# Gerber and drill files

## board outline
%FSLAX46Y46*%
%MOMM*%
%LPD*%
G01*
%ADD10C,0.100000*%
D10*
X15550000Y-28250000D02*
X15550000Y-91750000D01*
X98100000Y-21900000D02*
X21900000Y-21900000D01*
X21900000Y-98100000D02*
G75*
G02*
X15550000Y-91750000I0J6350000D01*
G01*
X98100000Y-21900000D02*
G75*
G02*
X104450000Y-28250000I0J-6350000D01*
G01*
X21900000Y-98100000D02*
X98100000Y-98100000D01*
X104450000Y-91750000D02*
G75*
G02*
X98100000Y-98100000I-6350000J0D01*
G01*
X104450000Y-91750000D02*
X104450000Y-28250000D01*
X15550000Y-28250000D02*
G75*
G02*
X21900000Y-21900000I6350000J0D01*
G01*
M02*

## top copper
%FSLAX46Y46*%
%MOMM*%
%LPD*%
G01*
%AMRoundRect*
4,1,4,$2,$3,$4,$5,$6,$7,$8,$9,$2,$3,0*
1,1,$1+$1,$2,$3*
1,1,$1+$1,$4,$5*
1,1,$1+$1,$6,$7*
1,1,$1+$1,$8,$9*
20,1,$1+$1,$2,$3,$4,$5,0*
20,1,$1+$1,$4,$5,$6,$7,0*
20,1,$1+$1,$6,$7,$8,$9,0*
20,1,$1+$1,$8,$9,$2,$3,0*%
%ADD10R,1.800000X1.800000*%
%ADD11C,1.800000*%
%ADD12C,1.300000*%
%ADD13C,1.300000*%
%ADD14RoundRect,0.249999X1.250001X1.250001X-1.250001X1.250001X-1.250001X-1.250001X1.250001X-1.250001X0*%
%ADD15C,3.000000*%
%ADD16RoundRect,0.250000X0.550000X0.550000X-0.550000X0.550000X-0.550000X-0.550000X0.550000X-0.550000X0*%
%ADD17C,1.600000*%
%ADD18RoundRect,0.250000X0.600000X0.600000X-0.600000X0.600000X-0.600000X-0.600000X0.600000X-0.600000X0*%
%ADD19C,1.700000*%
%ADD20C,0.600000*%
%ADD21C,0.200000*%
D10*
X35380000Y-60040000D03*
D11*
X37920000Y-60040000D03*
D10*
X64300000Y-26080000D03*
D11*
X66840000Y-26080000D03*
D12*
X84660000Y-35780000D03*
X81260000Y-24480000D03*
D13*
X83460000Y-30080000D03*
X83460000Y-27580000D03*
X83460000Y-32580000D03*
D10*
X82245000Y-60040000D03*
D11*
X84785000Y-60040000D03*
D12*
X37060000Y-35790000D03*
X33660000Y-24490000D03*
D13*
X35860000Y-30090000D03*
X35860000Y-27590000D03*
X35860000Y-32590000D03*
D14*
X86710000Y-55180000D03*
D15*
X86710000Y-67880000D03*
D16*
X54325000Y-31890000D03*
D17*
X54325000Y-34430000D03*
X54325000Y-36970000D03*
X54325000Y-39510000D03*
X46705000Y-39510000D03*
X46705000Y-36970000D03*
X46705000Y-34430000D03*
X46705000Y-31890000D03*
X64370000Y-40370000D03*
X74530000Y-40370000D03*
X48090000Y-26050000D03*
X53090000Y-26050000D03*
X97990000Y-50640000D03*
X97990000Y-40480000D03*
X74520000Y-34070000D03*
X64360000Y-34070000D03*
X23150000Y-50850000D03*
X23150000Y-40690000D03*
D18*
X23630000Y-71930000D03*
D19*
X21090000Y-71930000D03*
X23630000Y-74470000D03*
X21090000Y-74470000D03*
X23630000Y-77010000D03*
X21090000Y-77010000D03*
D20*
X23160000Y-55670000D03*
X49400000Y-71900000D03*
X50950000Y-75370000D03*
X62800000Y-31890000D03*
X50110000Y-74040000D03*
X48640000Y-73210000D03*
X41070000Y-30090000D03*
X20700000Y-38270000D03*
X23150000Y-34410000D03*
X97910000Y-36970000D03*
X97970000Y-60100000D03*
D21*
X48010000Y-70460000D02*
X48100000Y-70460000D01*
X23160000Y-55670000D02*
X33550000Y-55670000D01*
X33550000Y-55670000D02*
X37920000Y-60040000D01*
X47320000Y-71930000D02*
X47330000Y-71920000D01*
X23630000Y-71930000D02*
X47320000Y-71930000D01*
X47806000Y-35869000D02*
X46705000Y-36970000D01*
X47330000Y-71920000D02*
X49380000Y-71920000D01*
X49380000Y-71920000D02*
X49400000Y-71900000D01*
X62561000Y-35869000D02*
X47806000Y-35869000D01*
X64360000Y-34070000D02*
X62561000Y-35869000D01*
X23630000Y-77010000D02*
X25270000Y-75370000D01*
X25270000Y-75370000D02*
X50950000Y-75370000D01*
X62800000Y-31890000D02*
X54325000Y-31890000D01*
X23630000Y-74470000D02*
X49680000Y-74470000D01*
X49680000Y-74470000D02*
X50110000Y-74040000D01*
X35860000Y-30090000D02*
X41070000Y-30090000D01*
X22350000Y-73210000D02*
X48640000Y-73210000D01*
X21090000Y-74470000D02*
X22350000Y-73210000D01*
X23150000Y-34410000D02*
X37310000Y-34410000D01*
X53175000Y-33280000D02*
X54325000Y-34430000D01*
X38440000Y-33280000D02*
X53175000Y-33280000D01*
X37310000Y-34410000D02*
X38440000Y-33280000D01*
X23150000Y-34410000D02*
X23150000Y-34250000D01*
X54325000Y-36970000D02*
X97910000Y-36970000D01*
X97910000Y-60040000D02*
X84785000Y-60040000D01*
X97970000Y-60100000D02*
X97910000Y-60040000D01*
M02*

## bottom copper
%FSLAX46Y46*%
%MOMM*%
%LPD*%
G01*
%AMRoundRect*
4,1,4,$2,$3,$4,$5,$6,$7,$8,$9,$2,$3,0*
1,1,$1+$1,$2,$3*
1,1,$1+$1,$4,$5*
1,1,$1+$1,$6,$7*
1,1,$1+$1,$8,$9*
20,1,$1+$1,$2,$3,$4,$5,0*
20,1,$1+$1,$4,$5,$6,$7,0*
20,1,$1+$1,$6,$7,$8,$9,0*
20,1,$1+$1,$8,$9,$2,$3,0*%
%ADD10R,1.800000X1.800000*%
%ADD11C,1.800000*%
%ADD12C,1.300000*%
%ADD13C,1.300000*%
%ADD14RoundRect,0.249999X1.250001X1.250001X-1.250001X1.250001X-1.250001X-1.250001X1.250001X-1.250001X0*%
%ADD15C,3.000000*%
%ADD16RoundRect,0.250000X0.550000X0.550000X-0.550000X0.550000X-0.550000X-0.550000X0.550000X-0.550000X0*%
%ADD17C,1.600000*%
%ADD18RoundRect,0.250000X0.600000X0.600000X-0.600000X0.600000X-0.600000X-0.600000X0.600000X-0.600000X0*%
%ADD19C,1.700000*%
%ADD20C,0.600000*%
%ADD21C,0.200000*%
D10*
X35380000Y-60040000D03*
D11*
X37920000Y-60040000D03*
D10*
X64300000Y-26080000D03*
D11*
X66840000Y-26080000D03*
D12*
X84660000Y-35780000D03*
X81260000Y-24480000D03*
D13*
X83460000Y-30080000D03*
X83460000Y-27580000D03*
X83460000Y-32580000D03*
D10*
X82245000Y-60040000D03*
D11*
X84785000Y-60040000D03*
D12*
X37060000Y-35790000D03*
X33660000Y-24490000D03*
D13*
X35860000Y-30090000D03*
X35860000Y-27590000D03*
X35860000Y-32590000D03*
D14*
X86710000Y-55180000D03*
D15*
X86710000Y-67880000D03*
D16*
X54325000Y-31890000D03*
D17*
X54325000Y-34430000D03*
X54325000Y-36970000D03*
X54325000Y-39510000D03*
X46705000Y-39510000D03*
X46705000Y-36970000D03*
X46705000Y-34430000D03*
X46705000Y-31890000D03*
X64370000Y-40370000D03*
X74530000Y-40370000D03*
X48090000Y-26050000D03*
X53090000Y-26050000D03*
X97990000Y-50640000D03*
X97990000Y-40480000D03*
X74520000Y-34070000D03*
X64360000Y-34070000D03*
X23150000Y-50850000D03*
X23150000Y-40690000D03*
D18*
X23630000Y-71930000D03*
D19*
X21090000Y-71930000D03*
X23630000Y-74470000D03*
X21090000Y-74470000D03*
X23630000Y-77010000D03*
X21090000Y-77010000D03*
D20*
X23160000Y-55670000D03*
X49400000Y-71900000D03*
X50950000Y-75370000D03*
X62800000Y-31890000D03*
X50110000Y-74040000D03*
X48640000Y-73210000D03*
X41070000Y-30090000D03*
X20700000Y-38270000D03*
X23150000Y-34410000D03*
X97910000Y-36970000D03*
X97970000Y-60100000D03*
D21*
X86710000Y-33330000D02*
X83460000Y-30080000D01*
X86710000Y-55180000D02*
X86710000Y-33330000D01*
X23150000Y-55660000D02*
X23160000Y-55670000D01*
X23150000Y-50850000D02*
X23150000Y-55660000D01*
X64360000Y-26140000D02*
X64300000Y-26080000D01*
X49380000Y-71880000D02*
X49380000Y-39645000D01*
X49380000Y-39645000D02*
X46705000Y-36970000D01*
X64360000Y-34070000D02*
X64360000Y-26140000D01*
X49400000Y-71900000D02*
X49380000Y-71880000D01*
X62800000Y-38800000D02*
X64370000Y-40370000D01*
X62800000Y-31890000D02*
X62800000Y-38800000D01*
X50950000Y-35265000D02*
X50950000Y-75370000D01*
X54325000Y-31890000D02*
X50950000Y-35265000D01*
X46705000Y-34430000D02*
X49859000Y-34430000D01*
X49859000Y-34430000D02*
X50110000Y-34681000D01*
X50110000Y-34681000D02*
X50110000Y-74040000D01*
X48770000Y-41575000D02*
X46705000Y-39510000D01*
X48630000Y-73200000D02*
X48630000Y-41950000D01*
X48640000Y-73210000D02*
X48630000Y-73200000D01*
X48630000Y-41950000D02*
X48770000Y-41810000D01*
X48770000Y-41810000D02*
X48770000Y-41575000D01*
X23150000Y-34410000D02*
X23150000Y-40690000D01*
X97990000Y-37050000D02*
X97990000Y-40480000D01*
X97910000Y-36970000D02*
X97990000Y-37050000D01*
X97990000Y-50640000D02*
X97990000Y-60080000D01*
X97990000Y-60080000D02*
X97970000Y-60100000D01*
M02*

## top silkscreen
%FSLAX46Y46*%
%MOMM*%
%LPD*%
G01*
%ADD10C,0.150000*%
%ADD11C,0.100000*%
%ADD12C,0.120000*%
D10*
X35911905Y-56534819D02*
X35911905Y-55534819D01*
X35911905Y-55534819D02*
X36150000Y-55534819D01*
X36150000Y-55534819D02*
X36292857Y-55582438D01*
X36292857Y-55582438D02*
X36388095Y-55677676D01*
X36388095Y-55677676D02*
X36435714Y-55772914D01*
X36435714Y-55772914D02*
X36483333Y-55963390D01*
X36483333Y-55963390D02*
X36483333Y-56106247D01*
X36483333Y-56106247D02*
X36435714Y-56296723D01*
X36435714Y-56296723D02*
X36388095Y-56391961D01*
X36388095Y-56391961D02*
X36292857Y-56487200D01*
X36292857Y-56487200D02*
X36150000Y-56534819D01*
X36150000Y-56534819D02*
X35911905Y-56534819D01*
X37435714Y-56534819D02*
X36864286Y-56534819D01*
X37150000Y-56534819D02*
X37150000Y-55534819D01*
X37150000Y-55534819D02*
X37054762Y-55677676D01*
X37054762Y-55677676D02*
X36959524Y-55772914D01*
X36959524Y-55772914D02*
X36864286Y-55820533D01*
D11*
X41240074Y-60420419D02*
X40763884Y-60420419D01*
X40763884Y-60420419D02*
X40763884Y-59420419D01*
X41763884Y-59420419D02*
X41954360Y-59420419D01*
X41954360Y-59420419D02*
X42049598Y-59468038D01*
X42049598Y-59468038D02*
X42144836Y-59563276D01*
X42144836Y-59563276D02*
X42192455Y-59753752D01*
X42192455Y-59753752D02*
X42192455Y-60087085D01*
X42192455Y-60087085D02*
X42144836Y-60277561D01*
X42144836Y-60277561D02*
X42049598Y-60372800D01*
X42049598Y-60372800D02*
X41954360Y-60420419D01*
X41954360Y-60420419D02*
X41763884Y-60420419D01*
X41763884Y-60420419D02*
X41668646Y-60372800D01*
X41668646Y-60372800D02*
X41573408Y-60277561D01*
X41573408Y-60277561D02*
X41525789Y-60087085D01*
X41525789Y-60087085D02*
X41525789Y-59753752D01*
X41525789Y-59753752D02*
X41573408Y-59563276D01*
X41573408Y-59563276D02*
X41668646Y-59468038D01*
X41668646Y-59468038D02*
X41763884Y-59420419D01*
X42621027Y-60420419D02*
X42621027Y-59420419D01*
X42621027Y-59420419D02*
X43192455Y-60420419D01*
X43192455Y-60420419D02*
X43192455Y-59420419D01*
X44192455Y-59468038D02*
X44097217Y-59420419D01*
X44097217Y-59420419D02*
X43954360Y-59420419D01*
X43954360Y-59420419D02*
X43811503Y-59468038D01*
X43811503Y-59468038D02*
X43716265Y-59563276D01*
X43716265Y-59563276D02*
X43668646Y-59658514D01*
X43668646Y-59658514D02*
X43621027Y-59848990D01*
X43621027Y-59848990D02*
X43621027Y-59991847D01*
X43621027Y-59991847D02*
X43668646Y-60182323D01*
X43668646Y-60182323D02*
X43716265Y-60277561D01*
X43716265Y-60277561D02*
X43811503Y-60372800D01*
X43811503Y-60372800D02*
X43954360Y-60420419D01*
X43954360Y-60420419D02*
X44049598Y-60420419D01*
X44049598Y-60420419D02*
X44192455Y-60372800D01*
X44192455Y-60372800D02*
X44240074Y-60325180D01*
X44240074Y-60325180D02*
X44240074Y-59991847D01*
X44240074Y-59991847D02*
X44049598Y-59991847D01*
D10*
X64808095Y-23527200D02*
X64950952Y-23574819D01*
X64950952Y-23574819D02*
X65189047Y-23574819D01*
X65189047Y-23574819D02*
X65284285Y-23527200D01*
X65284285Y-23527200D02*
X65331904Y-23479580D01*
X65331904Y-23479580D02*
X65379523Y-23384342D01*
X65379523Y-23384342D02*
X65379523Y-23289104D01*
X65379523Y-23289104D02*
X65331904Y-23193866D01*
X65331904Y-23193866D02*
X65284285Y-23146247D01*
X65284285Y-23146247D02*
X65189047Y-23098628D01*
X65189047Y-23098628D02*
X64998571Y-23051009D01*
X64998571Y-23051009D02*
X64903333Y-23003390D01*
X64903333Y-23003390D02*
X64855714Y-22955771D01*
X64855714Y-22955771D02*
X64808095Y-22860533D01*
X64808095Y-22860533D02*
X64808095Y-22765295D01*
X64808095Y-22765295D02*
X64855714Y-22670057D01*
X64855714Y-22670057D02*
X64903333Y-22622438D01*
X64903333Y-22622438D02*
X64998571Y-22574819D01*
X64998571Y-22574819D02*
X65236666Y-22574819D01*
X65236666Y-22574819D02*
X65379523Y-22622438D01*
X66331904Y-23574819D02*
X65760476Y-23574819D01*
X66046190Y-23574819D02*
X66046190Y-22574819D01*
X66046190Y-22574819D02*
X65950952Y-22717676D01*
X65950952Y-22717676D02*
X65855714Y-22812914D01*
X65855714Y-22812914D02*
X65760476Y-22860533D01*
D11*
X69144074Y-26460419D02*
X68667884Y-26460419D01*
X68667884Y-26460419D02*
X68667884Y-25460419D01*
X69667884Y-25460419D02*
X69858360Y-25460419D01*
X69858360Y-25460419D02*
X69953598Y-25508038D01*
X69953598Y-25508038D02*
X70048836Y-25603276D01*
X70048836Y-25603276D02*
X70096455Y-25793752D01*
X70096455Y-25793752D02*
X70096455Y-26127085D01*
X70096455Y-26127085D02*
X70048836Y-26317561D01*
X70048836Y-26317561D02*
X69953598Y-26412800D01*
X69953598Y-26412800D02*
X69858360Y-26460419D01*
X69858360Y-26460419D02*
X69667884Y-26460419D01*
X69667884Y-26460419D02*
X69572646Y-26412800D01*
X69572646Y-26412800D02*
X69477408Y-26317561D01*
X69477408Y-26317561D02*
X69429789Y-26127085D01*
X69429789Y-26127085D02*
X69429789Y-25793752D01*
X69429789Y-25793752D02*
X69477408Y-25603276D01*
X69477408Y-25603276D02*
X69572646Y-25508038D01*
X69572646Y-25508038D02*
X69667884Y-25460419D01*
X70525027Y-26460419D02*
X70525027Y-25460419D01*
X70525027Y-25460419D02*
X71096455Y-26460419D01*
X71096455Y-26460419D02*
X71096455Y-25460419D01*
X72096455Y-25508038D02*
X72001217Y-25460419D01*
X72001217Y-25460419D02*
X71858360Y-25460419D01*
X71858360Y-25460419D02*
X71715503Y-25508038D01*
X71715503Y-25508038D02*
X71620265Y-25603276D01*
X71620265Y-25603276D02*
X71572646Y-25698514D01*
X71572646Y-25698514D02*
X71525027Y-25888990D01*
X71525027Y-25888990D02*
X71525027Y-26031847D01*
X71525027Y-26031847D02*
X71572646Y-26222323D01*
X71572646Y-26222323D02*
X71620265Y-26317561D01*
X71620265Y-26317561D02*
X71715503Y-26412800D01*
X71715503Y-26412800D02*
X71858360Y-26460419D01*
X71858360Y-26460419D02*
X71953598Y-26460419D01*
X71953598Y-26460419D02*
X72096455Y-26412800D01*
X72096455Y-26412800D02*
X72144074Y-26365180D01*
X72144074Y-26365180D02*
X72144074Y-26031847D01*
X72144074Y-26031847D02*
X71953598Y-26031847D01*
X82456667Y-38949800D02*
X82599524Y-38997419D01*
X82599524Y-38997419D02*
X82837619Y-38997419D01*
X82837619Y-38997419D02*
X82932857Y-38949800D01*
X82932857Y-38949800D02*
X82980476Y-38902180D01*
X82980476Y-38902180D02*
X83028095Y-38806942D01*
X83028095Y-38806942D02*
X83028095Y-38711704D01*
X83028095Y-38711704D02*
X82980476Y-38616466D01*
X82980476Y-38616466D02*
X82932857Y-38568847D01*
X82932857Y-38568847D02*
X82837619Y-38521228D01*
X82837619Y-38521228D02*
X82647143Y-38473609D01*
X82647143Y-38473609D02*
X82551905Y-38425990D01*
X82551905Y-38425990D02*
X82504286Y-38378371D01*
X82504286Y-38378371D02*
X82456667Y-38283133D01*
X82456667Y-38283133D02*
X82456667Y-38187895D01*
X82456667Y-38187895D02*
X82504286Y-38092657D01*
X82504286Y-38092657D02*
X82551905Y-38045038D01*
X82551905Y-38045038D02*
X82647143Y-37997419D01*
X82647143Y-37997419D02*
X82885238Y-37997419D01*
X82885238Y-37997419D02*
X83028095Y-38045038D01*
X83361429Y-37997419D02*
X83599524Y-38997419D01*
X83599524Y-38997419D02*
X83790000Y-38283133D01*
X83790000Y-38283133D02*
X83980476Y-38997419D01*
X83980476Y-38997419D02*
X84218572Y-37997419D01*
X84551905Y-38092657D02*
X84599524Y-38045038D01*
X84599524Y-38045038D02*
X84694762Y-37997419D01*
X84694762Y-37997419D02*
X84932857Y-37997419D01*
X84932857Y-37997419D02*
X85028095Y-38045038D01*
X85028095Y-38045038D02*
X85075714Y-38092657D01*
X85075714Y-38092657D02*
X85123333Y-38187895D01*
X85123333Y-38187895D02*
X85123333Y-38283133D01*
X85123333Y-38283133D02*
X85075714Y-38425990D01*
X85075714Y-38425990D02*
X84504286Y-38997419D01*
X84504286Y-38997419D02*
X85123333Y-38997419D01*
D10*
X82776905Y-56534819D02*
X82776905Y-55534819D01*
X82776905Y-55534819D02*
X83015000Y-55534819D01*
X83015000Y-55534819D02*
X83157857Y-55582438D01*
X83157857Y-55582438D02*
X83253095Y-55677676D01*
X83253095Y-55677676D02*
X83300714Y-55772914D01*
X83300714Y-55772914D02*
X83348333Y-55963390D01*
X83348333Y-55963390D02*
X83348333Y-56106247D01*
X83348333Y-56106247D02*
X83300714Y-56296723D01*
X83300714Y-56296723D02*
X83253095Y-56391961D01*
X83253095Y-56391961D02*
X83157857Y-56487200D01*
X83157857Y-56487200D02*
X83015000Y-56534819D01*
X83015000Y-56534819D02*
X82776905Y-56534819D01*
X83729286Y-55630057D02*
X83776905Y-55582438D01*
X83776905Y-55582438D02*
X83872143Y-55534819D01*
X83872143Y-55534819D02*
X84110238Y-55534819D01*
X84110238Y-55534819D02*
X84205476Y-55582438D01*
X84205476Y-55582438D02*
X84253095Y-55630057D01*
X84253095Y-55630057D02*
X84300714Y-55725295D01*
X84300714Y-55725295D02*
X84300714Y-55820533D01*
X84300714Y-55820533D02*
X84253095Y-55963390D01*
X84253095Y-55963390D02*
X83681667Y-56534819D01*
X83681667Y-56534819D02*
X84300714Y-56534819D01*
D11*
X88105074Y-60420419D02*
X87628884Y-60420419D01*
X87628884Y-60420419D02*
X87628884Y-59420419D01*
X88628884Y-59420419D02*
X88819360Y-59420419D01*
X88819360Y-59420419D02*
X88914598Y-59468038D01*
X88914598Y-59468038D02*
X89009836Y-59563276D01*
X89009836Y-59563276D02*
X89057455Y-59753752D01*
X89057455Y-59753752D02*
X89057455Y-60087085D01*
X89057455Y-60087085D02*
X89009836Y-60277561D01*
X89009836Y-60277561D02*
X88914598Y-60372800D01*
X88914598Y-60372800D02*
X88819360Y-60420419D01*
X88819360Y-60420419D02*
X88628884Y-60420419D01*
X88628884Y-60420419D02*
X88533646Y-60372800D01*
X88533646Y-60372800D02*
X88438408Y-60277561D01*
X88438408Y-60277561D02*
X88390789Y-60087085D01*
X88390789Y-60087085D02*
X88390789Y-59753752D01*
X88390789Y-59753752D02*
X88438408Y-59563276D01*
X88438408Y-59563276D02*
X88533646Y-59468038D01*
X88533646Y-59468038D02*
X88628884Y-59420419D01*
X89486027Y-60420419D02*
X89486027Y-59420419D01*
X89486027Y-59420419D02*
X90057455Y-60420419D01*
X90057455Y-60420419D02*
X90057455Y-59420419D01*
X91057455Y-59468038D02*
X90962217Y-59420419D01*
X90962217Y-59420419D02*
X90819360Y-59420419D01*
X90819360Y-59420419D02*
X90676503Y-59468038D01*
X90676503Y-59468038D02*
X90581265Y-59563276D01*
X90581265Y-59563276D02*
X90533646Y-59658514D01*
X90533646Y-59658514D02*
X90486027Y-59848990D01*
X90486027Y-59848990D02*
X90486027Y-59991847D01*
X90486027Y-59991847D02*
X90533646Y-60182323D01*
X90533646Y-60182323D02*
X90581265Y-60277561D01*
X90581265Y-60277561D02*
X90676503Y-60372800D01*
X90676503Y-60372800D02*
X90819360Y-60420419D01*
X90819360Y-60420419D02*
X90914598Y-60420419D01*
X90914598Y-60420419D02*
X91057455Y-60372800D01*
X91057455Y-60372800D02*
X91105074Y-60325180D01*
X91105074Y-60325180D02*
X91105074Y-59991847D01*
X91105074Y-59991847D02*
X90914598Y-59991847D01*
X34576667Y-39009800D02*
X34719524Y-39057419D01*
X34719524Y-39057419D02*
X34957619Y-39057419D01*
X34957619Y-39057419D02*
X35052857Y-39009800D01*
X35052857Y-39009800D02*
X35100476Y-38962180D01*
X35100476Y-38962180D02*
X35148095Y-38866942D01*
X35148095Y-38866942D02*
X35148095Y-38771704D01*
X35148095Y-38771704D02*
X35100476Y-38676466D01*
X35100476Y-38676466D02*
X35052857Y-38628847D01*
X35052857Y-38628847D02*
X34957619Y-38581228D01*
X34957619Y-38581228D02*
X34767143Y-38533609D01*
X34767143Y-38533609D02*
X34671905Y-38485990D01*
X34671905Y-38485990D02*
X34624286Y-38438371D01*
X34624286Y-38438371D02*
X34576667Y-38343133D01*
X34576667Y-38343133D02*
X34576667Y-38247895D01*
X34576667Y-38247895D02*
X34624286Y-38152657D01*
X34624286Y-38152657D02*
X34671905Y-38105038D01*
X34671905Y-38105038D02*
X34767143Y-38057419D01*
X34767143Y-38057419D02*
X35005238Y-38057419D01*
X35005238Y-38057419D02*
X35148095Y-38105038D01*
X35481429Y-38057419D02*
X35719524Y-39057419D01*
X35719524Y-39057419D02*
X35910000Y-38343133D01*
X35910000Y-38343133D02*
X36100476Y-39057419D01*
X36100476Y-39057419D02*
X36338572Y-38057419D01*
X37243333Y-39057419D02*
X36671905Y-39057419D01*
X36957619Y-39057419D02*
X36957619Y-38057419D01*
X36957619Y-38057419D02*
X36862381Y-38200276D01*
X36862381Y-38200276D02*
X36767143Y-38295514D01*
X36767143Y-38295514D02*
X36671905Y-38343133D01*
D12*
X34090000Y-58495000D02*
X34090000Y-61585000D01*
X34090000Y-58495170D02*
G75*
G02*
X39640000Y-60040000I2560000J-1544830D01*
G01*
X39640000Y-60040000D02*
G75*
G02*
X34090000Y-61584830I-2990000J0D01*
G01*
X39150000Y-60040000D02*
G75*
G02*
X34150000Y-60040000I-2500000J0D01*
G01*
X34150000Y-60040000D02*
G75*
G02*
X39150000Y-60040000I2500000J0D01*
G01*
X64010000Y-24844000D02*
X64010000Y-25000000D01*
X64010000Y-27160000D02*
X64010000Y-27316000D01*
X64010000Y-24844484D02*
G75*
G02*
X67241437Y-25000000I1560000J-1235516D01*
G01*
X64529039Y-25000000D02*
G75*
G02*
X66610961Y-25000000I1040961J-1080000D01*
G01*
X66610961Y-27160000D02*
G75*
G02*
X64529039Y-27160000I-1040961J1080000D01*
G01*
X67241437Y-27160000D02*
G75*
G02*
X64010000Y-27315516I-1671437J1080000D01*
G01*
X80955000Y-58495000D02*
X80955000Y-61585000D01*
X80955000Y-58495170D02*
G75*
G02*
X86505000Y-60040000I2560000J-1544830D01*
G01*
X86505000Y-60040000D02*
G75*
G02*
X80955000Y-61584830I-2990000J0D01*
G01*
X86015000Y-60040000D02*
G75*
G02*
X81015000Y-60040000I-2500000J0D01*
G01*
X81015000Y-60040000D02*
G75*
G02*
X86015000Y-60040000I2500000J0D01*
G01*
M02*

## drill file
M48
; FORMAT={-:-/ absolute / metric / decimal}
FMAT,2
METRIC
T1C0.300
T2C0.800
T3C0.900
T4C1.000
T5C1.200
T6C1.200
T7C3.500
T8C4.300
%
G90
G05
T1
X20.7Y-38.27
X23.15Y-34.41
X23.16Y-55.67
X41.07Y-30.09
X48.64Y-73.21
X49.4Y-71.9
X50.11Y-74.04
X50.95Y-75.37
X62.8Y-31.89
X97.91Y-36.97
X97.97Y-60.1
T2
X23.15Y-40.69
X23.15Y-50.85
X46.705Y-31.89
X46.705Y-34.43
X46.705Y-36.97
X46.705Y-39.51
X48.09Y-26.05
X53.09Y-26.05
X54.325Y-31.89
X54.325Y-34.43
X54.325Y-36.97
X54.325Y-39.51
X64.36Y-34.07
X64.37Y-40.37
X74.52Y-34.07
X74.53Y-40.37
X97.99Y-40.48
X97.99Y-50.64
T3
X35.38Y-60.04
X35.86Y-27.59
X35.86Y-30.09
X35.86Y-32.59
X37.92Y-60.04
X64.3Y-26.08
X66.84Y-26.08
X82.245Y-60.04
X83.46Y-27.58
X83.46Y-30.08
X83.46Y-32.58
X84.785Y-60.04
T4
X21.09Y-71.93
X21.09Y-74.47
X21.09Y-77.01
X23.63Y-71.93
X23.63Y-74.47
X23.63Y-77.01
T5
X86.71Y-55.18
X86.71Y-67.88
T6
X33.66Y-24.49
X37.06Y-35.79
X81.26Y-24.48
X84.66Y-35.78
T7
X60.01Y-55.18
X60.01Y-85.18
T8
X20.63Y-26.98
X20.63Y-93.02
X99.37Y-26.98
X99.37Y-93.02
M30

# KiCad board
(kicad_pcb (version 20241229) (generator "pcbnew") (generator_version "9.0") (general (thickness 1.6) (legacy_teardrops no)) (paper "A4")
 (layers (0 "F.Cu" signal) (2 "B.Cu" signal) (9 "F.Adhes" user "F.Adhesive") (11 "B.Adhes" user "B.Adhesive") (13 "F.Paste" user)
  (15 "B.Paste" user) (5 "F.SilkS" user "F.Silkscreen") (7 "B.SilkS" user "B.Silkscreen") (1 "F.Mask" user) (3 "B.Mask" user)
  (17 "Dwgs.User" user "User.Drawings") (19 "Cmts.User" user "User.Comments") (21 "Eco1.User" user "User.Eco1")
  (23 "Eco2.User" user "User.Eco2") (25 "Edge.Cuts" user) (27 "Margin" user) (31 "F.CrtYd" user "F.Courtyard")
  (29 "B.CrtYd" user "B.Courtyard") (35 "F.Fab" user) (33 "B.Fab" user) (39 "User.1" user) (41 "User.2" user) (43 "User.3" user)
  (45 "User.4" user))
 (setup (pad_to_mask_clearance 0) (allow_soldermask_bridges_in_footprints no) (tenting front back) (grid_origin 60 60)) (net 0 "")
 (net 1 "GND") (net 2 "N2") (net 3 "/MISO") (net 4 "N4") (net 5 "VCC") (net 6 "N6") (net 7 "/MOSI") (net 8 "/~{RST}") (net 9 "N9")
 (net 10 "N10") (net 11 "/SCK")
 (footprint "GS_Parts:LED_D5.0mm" (layer "F.Cu") (at 35.38 60.04)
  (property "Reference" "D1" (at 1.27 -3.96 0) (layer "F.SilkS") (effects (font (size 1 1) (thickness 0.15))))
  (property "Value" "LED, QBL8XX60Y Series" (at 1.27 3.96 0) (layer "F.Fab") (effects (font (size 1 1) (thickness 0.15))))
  (fp_line (start -1.29 -1.545) (end -1.29 1.545) (stroke (width 0.12) (type solid)) (layer "F.SilkS"))
  (fp_arc (start -1.29 -1.54483) (mid 2.071779 -2.880495) (end 4.26 0) (stroke (width 0.12) (type solid)) (layer "F.SilkS"))
  (fp_arc (start 4.26 0) (mid 2.071779 2.880495) (end -1.29 1.54483) (stroke (width 0.12) (type solid)) (layer "F.SilkS"))
  (fp_circle (center 1.27 0) (end 3.77 0) (stroke (width 0.12) (type solid)) (fill no) (layer "F.SilkS"))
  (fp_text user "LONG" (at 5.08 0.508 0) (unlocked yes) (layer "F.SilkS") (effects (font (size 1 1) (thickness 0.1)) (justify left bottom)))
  (pad "1" thru_hole rect (at 0 0) (size 1.8 1.8) (drill 0.9) (layers "*.Cu" "*.Mask") (remove_unused_layers no) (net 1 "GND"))
  (pad "2" thru_hole circle (at 2.54 0) (size 1.8 1.8) (drill 0.9) (layers "*.Cu" "*.Mask") (remove_unused_layers no) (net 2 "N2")))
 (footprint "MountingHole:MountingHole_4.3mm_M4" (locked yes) (layer "F.Cu") (at 20.63 26.98 90)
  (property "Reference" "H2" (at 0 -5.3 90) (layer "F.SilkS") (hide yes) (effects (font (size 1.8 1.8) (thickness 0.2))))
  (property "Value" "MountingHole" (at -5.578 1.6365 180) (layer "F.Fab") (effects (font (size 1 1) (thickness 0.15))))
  (pad "" np_thru_hole circle (at 0 0 90) (size 4.3 4.3) (drill 4.3) (layers "*.Cu" "*.Mask")))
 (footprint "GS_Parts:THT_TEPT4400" (layer "F.Cu") (at 64.3 26.08)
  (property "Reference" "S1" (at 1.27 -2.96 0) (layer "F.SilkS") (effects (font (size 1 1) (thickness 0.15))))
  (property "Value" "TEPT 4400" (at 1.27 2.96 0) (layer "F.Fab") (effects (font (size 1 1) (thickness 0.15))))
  (fp_line (start -0.29 -1.236) (end -0.29 -1.08) (stroke (width 0.12) (type solid)) (layer "F.SilkS"))
  (fp_line (start -0.29 1.08) (end -0.29 1.236) (stroke (width 0.12) (type solid)) (layer "F.SilkS"))
  (fp_arc (start -0.29 -1.235516) (mid 1.36566 -1.987699) (end 2.941437 -1.08) (stroke (width 0.12) (type solid)) (layer "F.SilkS"))
  (fp_arc (start 0.229039 -1.08) (mid 1.27 -1.5) (end 2.310961 -1.08) (stroke (width 0.12) (type solid)) (layer "F.SilkS"))
  (fp_arc (start 2.310961 1.08) (mid 1.27 1.5) (end 0.229039 1.08) (stroke (width 0.12) (type solid)) (layer "F.SilkS"))
  (fp_arc (start 2.941437 1.08) (mid 1.36566 1.987699) (end -0.29 1.235516) (stroke (width 0.12) (type solid)) (layer "F.SilkS"))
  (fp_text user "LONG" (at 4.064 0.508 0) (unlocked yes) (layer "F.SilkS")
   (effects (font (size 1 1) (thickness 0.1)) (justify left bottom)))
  (pad "1" thru_hole rect (at 0 0) (size 1.8 1.8) (drill 0.9) (layers "*.Cu" "*.Mask") (remove_unused_layers no) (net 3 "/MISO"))
  (pad "2" thru_hole circle (at 2.54 0) (size 1.8 1.8) (drill 0.9) (layers "*.Cu" "*.Mask") (remove_unused_layers no) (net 1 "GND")))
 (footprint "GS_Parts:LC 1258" (layer "F.Cu") (at 83.46 30.08 90)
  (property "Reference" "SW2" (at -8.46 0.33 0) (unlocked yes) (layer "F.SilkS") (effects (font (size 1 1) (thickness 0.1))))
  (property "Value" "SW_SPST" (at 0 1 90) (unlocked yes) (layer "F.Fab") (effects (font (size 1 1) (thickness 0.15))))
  (pad "" np_thru_hole circle (at -5.7 1.2 90) (size 1.3 1.3) (drill 1.2) (layers "*.Cu" "*.Mask"))
  (pad "" np_thru_hole circle (at 5.6 -2.2 90) (size 1.3 1.3) (drill 1.2) (layers "*.Cu" "*.Mask"))
  (pad "1" thru_hole circle (at 0 0 90) (size 1.3 1.3) (drill 0.9) (layers "*.Cu" "*.Mask") (remove_unused_layers no) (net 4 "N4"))
  (pad "2" thru_hole circle (at 2.5 0 90) (size 1.3 1.3) (drill 0.9) (layers "*.Cu" "*.Mask") (remove_unused_layers no) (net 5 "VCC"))
  (pad "3" thru_hole circle (at -2.5 0 90) (size 1.3 1.3) (drill 0.9) (layers "*.Cu" "*.Mask") (remove_unused_layers no)))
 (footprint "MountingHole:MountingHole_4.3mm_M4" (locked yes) (layer "F.Cu") (at 99.37 93.02 90)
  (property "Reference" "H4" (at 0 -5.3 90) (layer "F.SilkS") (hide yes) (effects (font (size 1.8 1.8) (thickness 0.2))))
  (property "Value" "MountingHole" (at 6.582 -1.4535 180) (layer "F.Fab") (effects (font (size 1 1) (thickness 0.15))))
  (pad "" np_thru_hole circle (at 0 0 90) (size 4.3 4.3) (drill 4.3) (layers "*.Cu" "*.Mask")))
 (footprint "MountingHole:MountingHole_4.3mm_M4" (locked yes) (layer "F.Cu") (at 99.37 26.98 90)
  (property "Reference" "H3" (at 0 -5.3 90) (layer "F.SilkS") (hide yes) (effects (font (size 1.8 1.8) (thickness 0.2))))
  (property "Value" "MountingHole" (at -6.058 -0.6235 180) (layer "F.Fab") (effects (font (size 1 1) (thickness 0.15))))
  (pad "" np_thru_hole circle (at 0 0 90) (size 4.3 4.3) (drill 4.3) (layers "*.Cu" "*.Mask")))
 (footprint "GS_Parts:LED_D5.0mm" (layer "F.Cu") (at 82.245 60.04)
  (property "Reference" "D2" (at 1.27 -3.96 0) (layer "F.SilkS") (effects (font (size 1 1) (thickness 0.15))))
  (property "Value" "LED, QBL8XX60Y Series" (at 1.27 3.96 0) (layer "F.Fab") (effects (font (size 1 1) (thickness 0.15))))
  (fp_line (start -1.29 -1.545) (end -1.29 1.545) (stroke (width 0.12) (type solid)) (layer "F.SilkS"))
  (fp_arc (start -1.29 -1.54483) (mid 2.071779 -2.880495) (end 4.26 0) (stroke (width 0.12) (type solid)) (layer "F.SilkS"))
  (fp_arc (start 4.26 0) (mid 2.071779 2.880495) (end -1.29 1.54483) (stroke (width 0.12) (type solid)) (layer "F.SilkS"))
  (fp_circle (center 1.27 0) (end 3.77 0) (stroke (width 0.12) (type solid)) (fill no) (layer "F.SilkS"))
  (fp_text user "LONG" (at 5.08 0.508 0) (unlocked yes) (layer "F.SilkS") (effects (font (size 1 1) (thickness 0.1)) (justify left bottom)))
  (pad "1" thru_hole rect (at 0 0) (size 1.8 1.8) (drill 0.9) (layers "*.Cu" "*.Mask") (remove_unused_layers no) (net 1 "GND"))
  (pad "2" thru_hole circle (at 2.54 0) (size 1.8 1.8) (drill 0.9) (layers "*.Cu" "*.Mask") (remove_unused_layers no) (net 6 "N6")))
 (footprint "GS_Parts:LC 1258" (layer "F.Cu") (at 35.86 30.09 90)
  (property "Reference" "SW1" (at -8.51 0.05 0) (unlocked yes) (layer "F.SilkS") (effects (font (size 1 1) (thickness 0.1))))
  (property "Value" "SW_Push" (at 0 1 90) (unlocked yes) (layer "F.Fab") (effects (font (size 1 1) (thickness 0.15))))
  (pad "" np_thru_hole circle (at -5.7 1.2 90) (size 1.3 1.3) (drill 1.2) (layers "*.Cu" "*.Mask"))
  (pad "" np_thru_hole circle (at 5.6 -2.2 90) (size 1.3 1.3) (drill 1.2) (layers "*.Cu" "*.Mask"))
  (pad "1" thru_hole circle (at 0 0 90) (size 1.3 1.3) (drill 0.9) (layers "*.Cu" "*.Mask") (remove_unused_layers no) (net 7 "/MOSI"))
  (pad "2" thru_hole circle (at 2.5 0 90) (size 1.3 1.3) (drill 0.9) (layers "*.Cu" "*.Mask") (remove_unused_layers no) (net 1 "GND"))
  (pad "3" thru_hole circle (at -2.5 0 90) (size 1.3 1.3) (drill 0.9) (layers "*.Cu" "*.Mask") (remove_unused_layers no)))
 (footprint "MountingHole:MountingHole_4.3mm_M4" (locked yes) (layer "F.Cu") (at 20.63 93.02 90)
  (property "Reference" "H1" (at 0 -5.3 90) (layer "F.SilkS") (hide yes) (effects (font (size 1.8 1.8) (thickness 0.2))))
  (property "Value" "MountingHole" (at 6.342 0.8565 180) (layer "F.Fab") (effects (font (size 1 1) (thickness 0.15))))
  (pad "" np_thru_hole circle (at 0 0 90) (size 4.3 4.3) (drill 4.3) (layers "*.Cu" "*.Mask")))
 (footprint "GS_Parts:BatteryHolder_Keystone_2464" (layer "B.Cu") (at 86.71 55.18 180)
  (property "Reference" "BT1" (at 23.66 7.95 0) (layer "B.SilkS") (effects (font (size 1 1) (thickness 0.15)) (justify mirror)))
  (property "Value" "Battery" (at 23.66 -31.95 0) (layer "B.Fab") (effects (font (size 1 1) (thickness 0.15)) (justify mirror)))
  (pad "" np_thru_hole circle (at 26.7 -30 180) (size 3.45 3.45) (drill 3.5) (layers "*.Cu" "*.Mask"))
  (pad "" np_thru_hole circle (at 26.7 0 180) (size 3.45 3.45) (drill 3.5) (layers "*.Cu" "*.Mask"))
  (pad "1" thru_hole roundrect (at 0 0 180) (size 3 3) (drill 1.2) (layers "*.Cu" "*.Mask") (remove_unused_layers no)
   (roundrect_rratio 0.083333) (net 4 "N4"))
  (pad "2" thru_hole circle (at 0 -12.7 180) (size 3 3) (drill 1.2) (layers "*.Cu" "*.Mask") (remove_unused_layers no) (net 1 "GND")))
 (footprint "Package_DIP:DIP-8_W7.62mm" (layer "B.Cu") (at 54.325 31.89 180)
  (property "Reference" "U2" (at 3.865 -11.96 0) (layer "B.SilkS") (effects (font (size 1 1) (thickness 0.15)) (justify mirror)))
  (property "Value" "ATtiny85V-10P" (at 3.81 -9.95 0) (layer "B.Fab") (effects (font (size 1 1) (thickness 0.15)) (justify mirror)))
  (pad "1" thru_hole roundrect (at 0 0 180) (size 1.6 1.6) (drill 0.8) (layers "*.Cu" "*.Mask") (remove_unused_layers no)
   (roundrect_rratio 0.15625) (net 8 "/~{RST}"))
  (pad "2" thru_hole circle (at 0 -2.54 180) (size 1.6 1.6) (drill 0.8) (layers "*.Cu" "*.Mask") (remove_unused_layers no) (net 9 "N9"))
  (pad "3" thru_hole circle (at 0 -5.08 180) (size 1.6 1.6) (drill 0.8) (layers "*.Cu" "*.Mask") (remove_unused_layers no) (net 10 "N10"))
  (pad "4" thru_hole circle (at 0 -7.62 180) (size 1.6 1.6) (drill 0.8) (layers "*.Cu" "*.Mask") (remove_unused_layers no) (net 1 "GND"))
  (pad "5" thru_hole circle (at 7.62 -7.62 180) (size 1.6 1.6) (drill 0.8) (layers "*.Cu" "*.Mask") (remove_unused_layers no)
   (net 7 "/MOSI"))
  (pad "6" thru_hole circle (at 7.62 -5.08 180) (size 1.6 1.6) (drill 0.8) (layers "*.Cu" "*.Mask") (remove_unused_layers no)
   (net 3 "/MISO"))
  (pad "7" thru_hole circle (at 7.62 -2.54 180) (size 1.6 1.6) (drill 0.8) (layers "*.Cu" "*.Mask") (remove_unused_layers no)
   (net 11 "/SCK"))
  (pad "8" thru_hole circle (at 7.62 0 180) (size 1.6 1.6) (drill 0.8) (layers "*.Cu" "*.Mask") (remove_unused_layers no) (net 5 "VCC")))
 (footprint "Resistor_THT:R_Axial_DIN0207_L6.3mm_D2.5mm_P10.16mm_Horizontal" (layer "B.Cu") (at 64.37 40.37)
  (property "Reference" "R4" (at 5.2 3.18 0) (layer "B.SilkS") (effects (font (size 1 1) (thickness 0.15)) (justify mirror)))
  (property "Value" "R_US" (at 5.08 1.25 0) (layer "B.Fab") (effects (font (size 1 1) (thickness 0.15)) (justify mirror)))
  (pad "1" thru_hole circle (at 0 0) (size 1.6 1.6) (drill 0.8) (layers "*.Cu" "*.Mask") (remove_unused_layers no) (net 8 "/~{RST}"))
  (pad "2" thru_hole circle (at 10.16 0) (size 1.6 1.6) (drill 0.8) (layers "*.Cu" "*.Mask") (remove_unused_layers no) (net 5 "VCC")))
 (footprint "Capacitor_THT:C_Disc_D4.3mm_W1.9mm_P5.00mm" (layer "B.Cu") (at 48.09 26.05)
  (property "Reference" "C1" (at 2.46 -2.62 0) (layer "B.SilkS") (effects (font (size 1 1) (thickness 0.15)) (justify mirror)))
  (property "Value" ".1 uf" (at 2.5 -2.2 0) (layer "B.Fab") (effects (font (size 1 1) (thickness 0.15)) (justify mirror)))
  (pad "1" thru_hole circle (at 0 0) (size 1.6 1.6) (drill 0.8) (layers "*.Cu" "*.Mask") (remove_unused_layers no) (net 5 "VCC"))
  (pad "2" thru_hole circle (at 5 0) (size 1.6 1.6) (drill 0.8) (layers "*.Cu" "*.Mask") (remove_unused_layers no) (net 1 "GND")))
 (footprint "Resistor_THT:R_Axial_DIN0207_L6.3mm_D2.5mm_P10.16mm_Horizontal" (layer "B.Cu") (at 97.99 50.64 90)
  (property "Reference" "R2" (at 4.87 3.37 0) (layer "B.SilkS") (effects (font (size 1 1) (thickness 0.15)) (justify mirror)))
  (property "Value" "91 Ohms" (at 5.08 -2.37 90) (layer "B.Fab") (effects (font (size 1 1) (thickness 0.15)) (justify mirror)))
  (pad "1" thru_hole circle (at 0 0 90) (size 1.6 1.6) (drill 0.8) (layers "*.Cu" "*.Mask") (remove_unused_layers no) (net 6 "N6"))
  (pad "2" thru_hole circle (at 10.16 0 90) (size 1.6 1.6) (drill 0.8) (layers "*.Cu" "*.Mask") (remove_unused_layers no) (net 10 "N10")))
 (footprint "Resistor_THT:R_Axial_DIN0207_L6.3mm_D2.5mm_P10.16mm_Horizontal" (layer "B.Cu") (at 74.52 34.07 180)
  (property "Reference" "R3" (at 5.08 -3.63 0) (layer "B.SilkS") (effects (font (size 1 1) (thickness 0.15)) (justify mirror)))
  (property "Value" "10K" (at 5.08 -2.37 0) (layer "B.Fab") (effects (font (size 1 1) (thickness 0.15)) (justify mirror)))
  (pad "1" thru_hole circle (at 0 0 180) (size 1.6 1.6) (drill 0.8) (layers "*.Cu" "*.Mask") (remove_unused_layers no) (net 5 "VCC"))
  (pad "2" thru_hole circle (at 10.16 0 180) (size 1.6 1.6) (drill 0.8) (layers "*.Cu" "*.Mask") (remove_unused_layers no) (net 3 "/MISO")))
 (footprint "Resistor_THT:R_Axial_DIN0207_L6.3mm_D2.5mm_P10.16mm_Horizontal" (layer "B.Cu") (at 23.15 50.85 90)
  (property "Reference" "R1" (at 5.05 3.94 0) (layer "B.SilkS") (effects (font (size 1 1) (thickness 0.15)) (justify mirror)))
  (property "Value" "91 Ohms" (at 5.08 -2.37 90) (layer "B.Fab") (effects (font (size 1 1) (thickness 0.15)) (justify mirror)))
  (pad "1" thru_hole circle (at 0 0 90) (size 1.6 1.6) (drill 0.8) (layers "*.Cu" "*.Mask") (remove_unused_layers no) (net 2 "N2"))
  (pad "2" thru_hole circle (at 10.16 0 90) (size 1.6 1.6) (drill 0.8) (layers "*.Cu" "*.Mask") (remove_unused_layers no) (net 9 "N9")))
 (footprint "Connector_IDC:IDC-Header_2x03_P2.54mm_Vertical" (layer "B.Cu") (at 23.63 71.93 180)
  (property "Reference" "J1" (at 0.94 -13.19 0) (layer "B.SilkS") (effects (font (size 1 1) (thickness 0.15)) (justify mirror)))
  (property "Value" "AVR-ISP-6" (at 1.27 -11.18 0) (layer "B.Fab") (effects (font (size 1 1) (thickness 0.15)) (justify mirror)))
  (pad "1" thru_hole roundrect (at 0 0 180) (size 1.7 1.7) (drill 1) (layers "*.Cu" "*.Mask") (remove_unused_layers no)
   (roundrect_rratio 0.147059) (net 3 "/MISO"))
  (pad "2" thru_hole circle (at 2.54 0 180) (size 1.7 1.7) (drill 1) (layers "*.Cu" "*.Mask") (remove_unused_layers no) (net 5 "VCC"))
  (pad "3" thru_hole circle (at 0 -2.54 180) (size 1.7 1.7) (drill 1) (layers "*.Cu" "*.Mask") (remove_unused_layers no) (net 11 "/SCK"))
  (pad "4" thru_hole circle (at 2.54 -2.54 180) (size 1.7 1.7) (drill 1) (layers "*.Cu" "*.Mask") (remove_unused_layers no) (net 7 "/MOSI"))
  (pad "5" thru_hole circle (at 0 -5.08 180) (size 1.7 1.7) (drill 1) (layers "*.Cu" "*.Mask") (remove_unused_layers no) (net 8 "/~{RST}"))
  (pad "6" thru_hole circle (at 2.54 -5.08 180) (size 1.7 1.7) (drill 1) (layers "*.Cu" "*.Mask") (remove_unused_layers no) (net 1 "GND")))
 (gr_line (start 15.55 28.25) (end 15.55 91.75) (stroke (width 0.1) (type default)) (locked yes) (layer "Edge.Cuts"))
 (gr_line (start 98.1 21.9) (end 21.9 21.9) (stroke (width 0.1) (type default)) (locked yes) (layer "Edge.Cuts"))
 (gr_arc (start 21.9 98.1) (mid 17.409872 96.240128) (end 15.55 91.75) (stroke (width 0.1) (type default)) (locked yes) (layer "Edge.Cuts"))
 (gr_arc (start 98.1 21.9) (mid 102.590128 23.759872) (end 104.45 28.25) (stroke (width 0.1) (type default)) (locked yes)
  (layer "Edge.Cuts"))
 (gr_line (start 21.9 98.1) (end 98.1 98.1) (stroke (width 0.1) (type default)) (locked yes) (layer "Edge.Cuts"))
 (gr_arc (start 104.45 91.75) (mid 102.590128 96.240128) (end 98.1 98.1) (stroke (width 0.1) (type default)) (locked yes)
  (layer "Edge.Cuts"))
 (gr_line (start 104.45 91.75) (end 104.45 28.25) (stroke (width 0.1) (type default)) (locked yes) (layer "Edge.Cuts"))
 (gr_arc (start 15.55 28.25) (mid 17.409872 23.759872) (end 21.9 21.9) (stroke (width 0.1) (type default)) (locked yes) (layer "Edge.Cuts"))
 (segment (start 86.71 33.33) (end 83.46 30.08) (width 0.2) (layer "B.Cu") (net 4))
 (segment (start 86.71 55.18) (end 86.71 33.33) (width 0.2) (layer "B.Cu") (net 4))
 (segment (start 48.01 70.46) (end 48.1 70.46) (width 0.2) (layer "F.Cu") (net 5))
 (segment (start 23.16 55.67) (end 33.55 55.67) (width 0.2) (layer "F.Cu") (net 2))
 (segment (start 33.55 55.67) (end 37.92 60.04) (width 0.2) (layer "F.Cu") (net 2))
 (via (at 23.16 55.67) (size 0.6) (drill 0.3) (layers "F.Cu" "B.Cu") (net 2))
 (segment (start 23.15 55.66) (end 23.16 55.67) (width 0.2) (layer "B.Cu") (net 2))
 (segment (start 23.15 50.85) (end 23.15 55.66) (width 0.2) (layer "B.Cu") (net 2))
 (segment (start 47.32 71.93) (end 47.33 71.92) (width 0.2) (layer "F.Cu") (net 3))
 (segment (start 23.63 71.93) (end 47.32 71.93) (width 0.2) (layer "F.Cu") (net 3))
 (segment (start 47.806 35.869) (end 46.705 36.97) (width 0.2) (layer "F.Cu") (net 3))
 (segment (start 47.33 71.92) (end 49.38 71.92) (width 0.2) (layer "F.Cu") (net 3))
 (segment (start 49.38 71.92) (end 49.4 71.9) (width 0.2) (layer "F.Cu") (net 3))
 (segment (start 62.561 35.869) (end 47.806 35.869) (width 0.2) (layer "F.Cu") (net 3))
 (segment (start 64.36 34.07) (end 62.561 35.869) (width 0.2) (layer "F.Cu") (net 3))
 (via (at 49.4 71.9) (size 0.6) (drill 0.3) (layers "F.Cu" "B.Cu") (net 3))
 (segment (start 64.36 26.14) (end 64.3 26.08) (width 0.2) (layer "B.Cu") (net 3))
 (segment (start 49.38 71.88) (end 49.38 39.645) (width 0.2) (layer "B.Cu") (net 3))
 (segment (start 49.38 39.645) (end 46.705 36.97) (width 0.2) (layer "B.Cu") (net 3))
 (segment (start 64.36 34.07) (end 64.36 26.14) (width 0.2) (layer "B.Cu") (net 3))
 (segment (start 49.4 71.9) (end 49.38 71.88) (width 0.2) (layer "B.Cu") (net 3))
 (segment (start 23.63 77.01) (end 25.27 75.37) (width 0.2) (layer "F.Cu") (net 8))
 (segment (start 25.27 75.37) (end 50.95 75.37) (width 0.2) (layer "F.Cu") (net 8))
 (segment (start 62.8 31.89) (end 54.325 31.89) (width 0.2) (layer "F.Cu") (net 8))
 (via (at 50.95 75.37) (size 0.6) (drill 0.3) (layers "F.Cu" "B.Cu") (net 8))
 (via (at 62.8 31.89) (size 0.6) (drill 0.3) (layers "F.Cu" "B.Cu") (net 8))
 (segment (start 62.8 38.8) (end 64.37 40.37) (width 0.2) (layer "B.Cu") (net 8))
 (segment (start 62.8 31.89) (end 62.8 38.8) (width 0.2) (layer "B.Cu") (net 8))
 (segment (start 50.95 35.265) (end 50.95 75.37) (width 0.2) (layer "B.Cu") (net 8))
 (segment (start 54.325 31.89) (end 50.95 35.265) (width 0.2) (layer "B.Cu") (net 8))
 (segment (start 23.63 74.47) (end 49.68 74.47) (width 0.2) (layer "F.Cu") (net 11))
 (segment (start 49.68 74.47) (end 50.11 74.04) (width 0.2) (layer "F.Cu") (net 11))
 (via (at 50.11 74.04) (size 0.6) (drill 0.3) (layers "F.Cu" "B.Cu") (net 11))
 (segment (start 46.705 34.43) (end 49.859 34.43) (width 0.2) (layer "B.Cu") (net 11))
 (segment (start 49.859 34.43) (end 50.11 34.681) (width 0.2) (layer "B.Cu") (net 11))
 (segment (start 50.11 34.681) (end 50.11 74.04) (width 0.2) (layer "B.Cu") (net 11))
 (segment (start 35.86 30.09) (end 41.07 30.09) (width 0.2) (layer "F.Cu") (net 7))
 (segment (start 22.35 73.21) (end 48.64 73.21) (width 0.2) (layer "F.Cu") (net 7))
 (segment (start 21.09 74.47) (end 22.35 73.21) (width 0.2) (layer "F.Cu") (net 7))
 (via (at 48.64 73.21) (size 0.6) (drill 0.3) (layers "F.Cu" "B.Cu") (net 7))
 (via (at 41.07 30.09) (size 0.6) (drill 0.3) (layers "F.Cu" "B.Cu") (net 7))
 (via (at 20.7 38.27) (size 0.6) (drill 0.3) (layers "F.Cu" "B.Cu") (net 7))
 (segment (start 48.77 41.575) (end 46.705 39.51) (width 0.2) (layer "B.Cu") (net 7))
 (segment (start 48.63 73.2) (end 48.63 41.95) (width 0.2) (layer "B.Cu") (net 7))
 (segment (start 48.64 73.21) (end 48.63 73.2) (width 0.2) (layer "B.Cu") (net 7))
 (segment (start 48.63 41.95) (end 48.77 41.81) (width 0.2) (layer "B.Cu") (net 7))
 (segment (start 48.77 41.81) (end 48.77 41.575) (width 0.2) (layer "B.Cu") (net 7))
 (segment (start 23.15 34.41) (end 37.31 34.41) (width 0.2) (layer "F.Cu") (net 9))
 (segment (start 53.175 33.28) (end 54.325 34.43) (width 0.2) (layer "F.Cu") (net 9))
 (segment (start 38.44 33.28) (end 53.175 33.28) (width 0.2) (layer "F.Cu") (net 9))
 (segment (start 37.31 34.41) (end 38.44 33.28) (width 0.2) (layer "F.Cu") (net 9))
 (segment (start 23.15 34.41) (end 23.15 34.25) (width 0.2) (layer "F.Cu") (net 9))
 (via (at 23.15 34.41) (size 0.6) (drill 0.3) (layers "F.Cu" "B.Cu") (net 9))
 (segment (start 23.15 34.41) (end 23.15 40.69) (width 0.2) (layer "B.Cu") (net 9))
 (segment (start 54.325 36.97) (end 97.91 36.97) (width 0.2) (layer "F.Cu") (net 10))
 (via (at 97.91 36.97) (size 0.6) (drill 0.3) (layers "F.Cu" "B.Cu") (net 10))
 (segment (start 97.99 37.05) (end 97.99 40.48) (width 0.2) (layer "B.Cu") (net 10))
 (segment (start 97.91 36.97) (end 97.99 37.05) (width 0.2) (layer "B.Cu") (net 10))
 (segment (start 97.91 60.04) (end 84.785 60.04) (width 0.2) (layer "F.Cu") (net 6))
 (segment (start 97.97 60.1) (end 97.91 60.04) (width 0.2) (layer "F.Cu") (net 6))
 (via (at 97.97 60.1) (size 0.6) (drill 0.3) (layers "F.Cu" "B.Cu") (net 6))
 (segment (start 97.99 50.64) (end 97.99 60.08) (width 0.2) (layer "B.Cu") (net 6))
 (segment (start 97.99 60.08) (end 97.97 60.1) (width 0.2) (layer "B.Cu") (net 6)))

